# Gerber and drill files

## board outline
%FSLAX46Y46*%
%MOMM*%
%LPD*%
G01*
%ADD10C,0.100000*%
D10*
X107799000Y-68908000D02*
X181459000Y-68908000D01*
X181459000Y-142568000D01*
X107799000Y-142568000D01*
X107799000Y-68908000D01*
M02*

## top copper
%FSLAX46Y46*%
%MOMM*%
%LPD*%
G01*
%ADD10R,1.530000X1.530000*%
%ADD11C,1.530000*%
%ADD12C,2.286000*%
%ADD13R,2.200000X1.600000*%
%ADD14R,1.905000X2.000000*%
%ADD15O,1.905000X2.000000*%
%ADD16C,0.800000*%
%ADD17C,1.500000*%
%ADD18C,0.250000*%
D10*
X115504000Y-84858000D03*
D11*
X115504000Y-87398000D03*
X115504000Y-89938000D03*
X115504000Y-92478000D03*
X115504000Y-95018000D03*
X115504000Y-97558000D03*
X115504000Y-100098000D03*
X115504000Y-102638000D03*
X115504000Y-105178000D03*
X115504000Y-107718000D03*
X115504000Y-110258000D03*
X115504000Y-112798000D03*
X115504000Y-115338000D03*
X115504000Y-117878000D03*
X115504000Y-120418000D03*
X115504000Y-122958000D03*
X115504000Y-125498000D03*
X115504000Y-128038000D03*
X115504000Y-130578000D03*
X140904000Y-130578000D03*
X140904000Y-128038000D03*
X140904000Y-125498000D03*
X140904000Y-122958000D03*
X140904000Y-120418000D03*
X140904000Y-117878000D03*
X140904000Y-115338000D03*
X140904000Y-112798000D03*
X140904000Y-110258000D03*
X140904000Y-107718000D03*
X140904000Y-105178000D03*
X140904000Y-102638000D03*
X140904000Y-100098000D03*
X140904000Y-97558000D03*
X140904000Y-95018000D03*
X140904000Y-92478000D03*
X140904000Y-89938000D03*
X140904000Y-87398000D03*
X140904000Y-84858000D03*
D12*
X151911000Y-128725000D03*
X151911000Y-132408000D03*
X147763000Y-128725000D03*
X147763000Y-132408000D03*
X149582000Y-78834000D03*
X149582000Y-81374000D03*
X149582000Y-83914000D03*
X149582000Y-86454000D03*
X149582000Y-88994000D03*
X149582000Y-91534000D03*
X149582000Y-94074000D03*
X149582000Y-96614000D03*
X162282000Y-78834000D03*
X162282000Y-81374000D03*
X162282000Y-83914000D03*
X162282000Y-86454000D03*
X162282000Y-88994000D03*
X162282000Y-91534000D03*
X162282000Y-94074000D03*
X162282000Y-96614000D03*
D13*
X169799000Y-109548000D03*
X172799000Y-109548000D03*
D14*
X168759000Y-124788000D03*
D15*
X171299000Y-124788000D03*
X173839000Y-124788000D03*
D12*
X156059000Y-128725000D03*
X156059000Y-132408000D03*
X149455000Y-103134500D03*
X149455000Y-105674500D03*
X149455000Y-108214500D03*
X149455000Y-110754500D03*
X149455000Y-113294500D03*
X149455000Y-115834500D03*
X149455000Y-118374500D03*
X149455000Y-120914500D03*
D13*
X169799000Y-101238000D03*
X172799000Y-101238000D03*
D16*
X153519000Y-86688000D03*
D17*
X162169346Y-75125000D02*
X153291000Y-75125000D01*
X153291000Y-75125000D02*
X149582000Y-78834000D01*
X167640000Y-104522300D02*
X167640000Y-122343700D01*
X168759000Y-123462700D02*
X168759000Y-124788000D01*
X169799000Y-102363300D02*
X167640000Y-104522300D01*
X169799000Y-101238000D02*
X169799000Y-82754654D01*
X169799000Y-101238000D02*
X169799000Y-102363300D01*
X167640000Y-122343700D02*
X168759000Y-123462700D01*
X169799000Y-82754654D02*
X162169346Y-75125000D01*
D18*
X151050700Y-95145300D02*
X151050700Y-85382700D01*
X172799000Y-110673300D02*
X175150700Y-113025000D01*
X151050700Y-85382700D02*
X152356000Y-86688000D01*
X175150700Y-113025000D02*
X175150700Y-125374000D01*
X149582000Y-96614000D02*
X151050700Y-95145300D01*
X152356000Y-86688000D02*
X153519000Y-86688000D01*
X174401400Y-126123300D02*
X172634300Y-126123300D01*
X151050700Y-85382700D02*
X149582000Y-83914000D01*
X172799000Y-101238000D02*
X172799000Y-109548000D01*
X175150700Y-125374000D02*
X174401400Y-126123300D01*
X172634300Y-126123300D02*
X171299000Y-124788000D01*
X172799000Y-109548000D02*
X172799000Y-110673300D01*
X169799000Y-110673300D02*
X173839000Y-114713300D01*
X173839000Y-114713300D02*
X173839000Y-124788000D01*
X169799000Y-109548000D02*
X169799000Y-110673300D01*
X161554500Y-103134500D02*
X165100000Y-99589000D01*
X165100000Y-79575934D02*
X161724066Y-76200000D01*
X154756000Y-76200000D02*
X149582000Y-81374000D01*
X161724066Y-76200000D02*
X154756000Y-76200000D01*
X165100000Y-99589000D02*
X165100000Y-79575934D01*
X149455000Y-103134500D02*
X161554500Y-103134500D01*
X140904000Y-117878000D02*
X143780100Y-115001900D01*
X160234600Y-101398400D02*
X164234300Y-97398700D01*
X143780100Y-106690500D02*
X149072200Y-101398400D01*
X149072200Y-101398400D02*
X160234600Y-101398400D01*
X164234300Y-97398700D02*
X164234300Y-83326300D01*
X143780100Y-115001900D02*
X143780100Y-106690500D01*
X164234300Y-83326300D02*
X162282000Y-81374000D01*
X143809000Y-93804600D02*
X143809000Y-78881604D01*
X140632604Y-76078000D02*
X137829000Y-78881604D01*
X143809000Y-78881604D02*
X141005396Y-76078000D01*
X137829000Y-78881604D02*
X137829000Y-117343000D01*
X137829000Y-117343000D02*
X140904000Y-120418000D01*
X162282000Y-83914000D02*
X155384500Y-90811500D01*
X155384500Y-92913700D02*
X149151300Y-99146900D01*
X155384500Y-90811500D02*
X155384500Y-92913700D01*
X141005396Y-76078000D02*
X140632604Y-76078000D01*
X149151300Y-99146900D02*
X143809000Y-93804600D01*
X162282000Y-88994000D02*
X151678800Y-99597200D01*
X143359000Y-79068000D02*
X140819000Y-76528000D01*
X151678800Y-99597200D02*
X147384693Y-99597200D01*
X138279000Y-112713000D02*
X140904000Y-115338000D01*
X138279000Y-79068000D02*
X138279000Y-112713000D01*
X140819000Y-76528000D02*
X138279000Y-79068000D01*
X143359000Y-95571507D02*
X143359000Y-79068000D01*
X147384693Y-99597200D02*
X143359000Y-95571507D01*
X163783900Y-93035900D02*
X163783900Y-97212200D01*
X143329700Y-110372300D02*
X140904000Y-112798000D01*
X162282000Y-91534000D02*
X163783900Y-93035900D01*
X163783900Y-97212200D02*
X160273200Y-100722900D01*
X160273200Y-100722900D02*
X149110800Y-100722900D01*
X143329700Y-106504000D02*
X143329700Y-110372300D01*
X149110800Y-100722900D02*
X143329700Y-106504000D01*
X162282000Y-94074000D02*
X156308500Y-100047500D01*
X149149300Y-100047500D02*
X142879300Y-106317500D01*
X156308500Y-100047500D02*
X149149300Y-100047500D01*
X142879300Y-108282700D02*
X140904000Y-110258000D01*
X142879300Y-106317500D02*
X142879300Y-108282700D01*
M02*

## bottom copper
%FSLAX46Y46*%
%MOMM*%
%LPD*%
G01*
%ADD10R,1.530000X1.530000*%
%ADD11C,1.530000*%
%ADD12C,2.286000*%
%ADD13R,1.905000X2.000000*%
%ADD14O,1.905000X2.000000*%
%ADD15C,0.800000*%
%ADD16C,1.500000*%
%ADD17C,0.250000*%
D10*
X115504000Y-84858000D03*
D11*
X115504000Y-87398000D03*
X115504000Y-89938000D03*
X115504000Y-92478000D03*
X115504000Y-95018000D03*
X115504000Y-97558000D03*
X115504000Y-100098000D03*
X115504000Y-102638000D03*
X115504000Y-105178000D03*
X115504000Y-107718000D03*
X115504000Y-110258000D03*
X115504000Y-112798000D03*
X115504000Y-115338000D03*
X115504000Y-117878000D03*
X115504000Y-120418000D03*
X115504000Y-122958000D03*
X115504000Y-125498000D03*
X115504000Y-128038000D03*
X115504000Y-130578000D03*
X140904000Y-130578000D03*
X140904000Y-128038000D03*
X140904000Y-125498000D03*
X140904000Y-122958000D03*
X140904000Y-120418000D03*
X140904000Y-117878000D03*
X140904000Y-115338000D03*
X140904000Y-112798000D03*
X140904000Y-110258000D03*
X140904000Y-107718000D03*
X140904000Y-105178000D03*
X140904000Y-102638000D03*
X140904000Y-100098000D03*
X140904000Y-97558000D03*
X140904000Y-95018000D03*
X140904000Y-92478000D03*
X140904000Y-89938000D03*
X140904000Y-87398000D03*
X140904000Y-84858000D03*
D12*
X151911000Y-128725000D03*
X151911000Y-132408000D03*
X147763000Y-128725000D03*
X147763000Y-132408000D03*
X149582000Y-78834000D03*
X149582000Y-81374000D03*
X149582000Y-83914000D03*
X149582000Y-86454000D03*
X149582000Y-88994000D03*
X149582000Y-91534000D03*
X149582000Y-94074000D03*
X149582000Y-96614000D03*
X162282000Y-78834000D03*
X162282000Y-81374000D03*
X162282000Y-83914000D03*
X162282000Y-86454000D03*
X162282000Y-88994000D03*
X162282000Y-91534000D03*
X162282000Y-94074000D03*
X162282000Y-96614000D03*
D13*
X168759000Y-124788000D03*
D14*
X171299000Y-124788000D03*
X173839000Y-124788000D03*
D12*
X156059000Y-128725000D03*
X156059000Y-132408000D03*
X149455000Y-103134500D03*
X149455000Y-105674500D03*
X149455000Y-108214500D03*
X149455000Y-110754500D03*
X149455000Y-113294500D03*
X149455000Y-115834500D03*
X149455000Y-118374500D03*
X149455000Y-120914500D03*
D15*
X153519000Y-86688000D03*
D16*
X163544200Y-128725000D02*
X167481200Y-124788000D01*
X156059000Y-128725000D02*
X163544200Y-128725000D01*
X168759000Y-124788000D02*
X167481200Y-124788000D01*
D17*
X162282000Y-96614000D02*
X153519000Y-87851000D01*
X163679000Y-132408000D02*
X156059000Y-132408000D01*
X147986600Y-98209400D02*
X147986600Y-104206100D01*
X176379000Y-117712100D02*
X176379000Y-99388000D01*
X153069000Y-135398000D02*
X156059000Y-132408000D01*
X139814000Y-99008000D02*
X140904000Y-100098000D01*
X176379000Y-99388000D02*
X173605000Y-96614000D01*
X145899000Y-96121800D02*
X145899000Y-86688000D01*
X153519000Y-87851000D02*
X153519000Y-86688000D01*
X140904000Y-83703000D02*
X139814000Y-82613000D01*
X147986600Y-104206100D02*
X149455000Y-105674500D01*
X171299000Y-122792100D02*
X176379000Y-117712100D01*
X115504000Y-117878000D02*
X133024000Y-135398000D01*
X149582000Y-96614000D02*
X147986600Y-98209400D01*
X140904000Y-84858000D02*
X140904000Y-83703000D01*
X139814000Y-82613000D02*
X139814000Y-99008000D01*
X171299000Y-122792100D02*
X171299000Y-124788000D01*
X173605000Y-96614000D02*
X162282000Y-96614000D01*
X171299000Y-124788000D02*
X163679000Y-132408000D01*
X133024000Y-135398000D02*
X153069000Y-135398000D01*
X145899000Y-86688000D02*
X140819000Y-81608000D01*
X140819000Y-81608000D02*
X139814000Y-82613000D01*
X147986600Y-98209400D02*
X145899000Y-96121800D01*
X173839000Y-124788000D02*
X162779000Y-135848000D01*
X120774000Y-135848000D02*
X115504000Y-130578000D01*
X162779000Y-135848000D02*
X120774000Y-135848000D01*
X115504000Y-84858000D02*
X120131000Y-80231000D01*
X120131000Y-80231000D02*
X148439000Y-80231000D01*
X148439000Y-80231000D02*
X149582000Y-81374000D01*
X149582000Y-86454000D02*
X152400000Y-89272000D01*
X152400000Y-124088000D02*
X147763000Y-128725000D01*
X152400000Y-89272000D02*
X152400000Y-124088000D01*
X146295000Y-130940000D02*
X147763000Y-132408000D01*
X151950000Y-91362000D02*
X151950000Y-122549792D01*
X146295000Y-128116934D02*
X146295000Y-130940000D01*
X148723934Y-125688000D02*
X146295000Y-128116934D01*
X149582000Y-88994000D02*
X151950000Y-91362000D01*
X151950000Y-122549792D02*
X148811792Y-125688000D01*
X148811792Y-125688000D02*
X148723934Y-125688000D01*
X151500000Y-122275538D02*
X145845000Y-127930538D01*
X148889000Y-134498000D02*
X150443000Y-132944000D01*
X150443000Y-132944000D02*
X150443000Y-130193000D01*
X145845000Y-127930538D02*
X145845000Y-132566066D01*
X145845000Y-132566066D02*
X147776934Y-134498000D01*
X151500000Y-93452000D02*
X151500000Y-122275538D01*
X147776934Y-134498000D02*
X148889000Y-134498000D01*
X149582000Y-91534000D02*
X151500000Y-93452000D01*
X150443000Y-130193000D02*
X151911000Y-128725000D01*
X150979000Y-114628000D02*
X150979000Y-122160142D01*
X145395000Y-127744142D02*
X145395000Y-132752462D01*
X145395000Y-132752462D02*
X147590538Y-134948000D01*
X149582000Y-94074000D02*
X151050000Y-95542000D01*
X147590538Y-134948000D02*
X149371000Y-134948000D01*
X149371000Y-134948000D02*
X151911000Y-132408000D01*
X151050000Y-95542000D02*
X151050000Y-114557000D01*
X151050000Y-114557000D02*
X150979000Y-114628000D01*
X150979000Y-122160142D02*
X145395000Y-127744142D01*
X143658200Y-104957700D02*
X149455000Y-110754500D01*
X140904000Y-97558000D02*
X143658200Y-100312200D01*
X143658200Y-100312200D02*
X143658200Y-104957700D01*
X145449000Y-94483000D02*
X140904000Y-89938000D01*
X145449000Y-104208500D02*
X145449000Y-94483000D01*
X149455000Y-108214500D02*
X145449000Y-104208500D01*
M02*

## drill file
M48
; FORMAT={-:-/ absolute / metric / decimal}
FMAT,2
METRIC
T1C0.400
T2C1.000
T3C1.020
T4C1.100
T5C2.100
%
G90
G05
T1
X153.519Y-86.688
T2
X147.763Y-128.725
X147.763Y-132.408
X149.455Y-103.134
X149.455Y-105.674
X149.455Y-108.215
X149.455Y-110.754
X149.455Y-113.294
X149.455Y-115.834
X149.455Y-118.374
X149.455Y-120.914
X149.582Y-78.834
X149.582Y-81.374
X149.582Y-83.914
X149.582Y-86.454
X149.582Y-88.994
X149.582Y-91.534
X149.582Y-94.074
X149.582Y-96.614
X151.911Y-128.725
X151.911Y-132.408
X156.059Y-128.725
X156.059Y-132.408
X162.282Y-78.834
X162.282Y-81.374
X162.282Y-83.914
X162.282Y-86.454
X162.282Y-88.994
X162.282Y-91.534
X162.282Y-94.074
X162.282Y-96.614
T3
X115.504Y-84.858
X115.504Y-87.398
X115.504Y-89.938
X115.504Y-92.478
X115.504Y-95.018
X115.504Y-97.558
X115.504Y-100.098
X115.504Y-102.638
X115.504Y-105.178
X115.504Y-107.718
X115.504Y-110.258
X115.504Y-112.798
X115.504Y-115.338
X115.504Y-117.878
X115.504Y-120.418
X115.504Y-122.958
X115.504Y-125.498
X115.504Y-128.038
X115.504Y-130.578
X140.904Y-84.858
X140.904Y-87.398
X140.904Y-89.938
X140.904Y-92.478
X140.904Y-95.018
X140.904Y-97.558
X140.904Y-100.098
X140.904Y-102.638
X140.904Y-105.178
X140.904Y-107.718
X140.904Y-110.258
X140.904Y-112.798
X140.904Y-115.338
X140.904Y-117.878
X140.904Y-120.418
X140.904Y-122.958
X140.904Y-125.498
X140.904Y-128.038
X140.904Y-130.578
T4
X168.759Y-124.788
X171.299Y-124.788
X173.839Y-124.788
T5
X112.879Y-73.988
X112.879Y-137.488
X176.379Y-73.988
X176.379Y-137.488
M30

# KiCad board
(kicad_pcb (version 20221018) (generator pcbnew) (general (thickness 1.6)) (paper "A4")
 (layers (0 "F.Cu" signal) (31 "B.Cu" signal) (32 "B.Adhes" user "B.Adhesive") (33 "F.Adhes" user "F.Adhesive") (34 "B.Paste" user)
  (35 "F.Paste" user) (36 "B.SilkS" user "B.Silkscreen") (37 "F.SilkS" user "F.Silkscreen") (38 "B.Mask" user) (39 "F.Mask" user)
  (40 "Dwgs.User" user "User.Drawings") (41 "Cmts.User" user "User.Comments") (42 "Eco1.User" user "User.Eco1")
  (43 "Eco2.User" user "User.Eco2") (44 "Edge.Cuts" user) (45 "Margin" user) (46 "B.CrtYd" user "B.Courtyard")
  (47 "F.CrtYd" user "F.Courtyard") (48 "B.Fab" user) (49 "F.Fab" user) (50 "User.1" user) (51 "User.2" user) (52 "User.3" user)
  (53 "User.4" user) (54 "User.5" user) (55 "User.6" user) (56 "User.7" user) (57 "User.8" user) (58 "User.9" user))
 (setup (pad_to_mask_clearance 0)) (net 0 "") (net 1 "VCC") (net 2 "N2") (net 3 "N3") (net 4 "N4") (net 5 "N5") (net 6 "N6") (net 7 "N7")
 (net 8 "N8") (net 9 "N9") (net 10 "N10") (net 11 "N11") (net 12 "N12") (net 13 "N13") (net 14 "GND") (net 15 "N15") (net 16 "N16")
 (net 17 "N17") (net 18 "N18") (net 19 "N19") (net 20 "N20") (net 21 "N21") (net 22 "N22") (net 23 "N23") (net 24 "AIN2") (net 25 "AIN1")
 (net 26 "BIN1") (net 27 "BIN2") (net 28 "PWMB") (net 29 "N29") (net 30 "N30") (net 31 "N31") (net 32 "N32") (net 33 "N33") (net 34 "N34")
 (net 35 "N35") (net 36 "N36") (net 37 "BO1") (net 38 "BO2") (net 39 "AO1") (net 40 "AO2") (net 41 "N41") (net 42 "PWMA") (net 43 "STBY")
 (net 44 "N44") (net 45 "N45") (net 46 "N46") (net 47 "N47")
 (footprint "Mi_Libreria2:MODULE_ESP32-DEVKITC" (layer "F.Cu") (at 128.204 107.708)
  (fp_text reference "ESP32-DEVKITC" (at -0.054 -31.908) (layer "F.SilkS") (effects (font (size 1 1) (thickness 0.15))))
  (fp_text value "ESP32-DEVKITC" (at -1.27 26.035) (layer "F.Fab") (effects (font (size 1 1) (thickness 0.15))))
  (pad "1" thru_hole rect (at -12.7 -22.85) (size 1.53 1.53) (drill 1.02) (layers "*.Cu" "*.Mask") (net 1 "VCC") (solder_mask_margin 0.102))
  (pad "2" thru_hole circle (at -12.7 -20.31) (size 1.53 1.53) (drill 1.02) (layers "*.Cu" "*.Mask") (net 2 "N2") (solder_mask_margin 0.102))
  (pad "3" thru_hole circle (at -12.7 -17.77) (size 1.53 1.53) (drill 1.02) (layers "*.Cu" "*.Mask") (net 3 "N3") (solder_mask_margin 0.102))
  (pad "4" thru_hole circle (at -12.7 -15.23) (size 1.53 1.53) (drill 1.02) (layers "*.Cu" "*.Mask") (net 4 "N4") (solder_mask_margin 0.102))
  (pad "5" thru_hole circle (at -12.7 -12.69) (size 1.53 1.53) (drill 1.02) (layers "*.Cu" "*.Mask") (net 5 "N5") (solder_mask_margin 0.102))
  (pad "6" thru_hole circle (at -12.7 -10.15) (size 1.53 1.53) (drill 1.02) (layers "*.Cu" "*.Mask") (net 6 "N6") (solder_mask_margin 0.102))
  (pad "7" thru_hole circle (at -12.7 -7.61) (size 1.53 1.53) (drill 1.02) (layers "*.Cu" "*.Mask") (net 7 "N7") (solder_mask_margin 0.102))
  (pad "8" thru_hole circle (at -12.7 -5.07) (size 1.53 1.53) (drill 1.02) (layers "*.Cu" "*.Mask") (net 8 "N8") (solder_mask_margin 0.102))
  (pad "9" thru_hole circle (at -12.7 -2.53) (size 1.53 1.53) (drill 1.02) (layers "*.Cu" "*.Mask") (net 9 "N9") (solder_mask_margin 0.102))
  (pad "10" thru_hole circle (at -12.7 0.01) (size 1.53 1.53) (drill 1.02) (layers "*.Cu" "*.Mask") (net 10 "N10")
   (solder_mask_margin 0.102))
  (pad "11" thru_hole circle (at -12.7 2.55) (size 1.53 1.53) (drill 1.02) (layers "*.Cu" "*.Mask") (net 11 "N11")
   (solder_mask_margin 0.102))
  (pad "12" thru_hole circle (at -12.7 5.09) (size 1.53 1.53) (drill 1.02) (layers "*.Cu" "*.Mask") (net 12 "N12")
   (solder_mask_margin 0.102))
  (pad "13" thru_hole circle (at -12.7 7.63) (size 1.53 1.53) (drill 1.02) (layers "*.Cu" "*.Mask") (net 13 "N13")
   (solder_mask_margin 0.102))
  (pad "14" thru_hole circle (at -12.7 10.17) (size 1.53 1.53) (drill 1.02) (layers "*.Cu" "*.Mask") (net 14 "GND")
   (solder_mask_margin 0.102))
  (pad "15" thru_hole circle (at -12.7 12.71) (size 1.53 1.53) (drill 1.02) (layers "*.Cu" "*.Mask") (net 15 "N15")
   (solder_mask_margin 0.102))
  (pad "16" thru_hole circle (at -12.7 15.25) (size 1.53 1.53) (drill 1.02) (layers "*.Cu" "*.Mask") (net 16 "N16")
   (solder_mask_margin 0.102))
  (pad "17" thru_hole circle (at -12.7 17.79) (size 1.53 1.53) (drill 1.02) (layers "*.Cu" "*.Mask") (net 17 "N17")
   (solder_mask_margin 0.102))
  (pad "18" thru_hole circle (at -12.7 20.33) (size 1.53 1.53) (drill 1.02) (layers "*.Cu" "*.Mask") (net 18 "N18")
   (solder_mask_margin 0.102))
  (pad "19" thru_hole circle (at -12.7 22.87) (size 1.53 1.53) (drill 1.02) (layers "*.Cu" "*.Mask") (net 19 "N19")
   (solder_mask_margin 0.102))
  (pad "20" thru_hole circle (at 12.7 22.87) (size 1.53 1.53) (drill 1.02) (layers "*.Cu" "*.Mask") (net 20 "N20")
   (solder_mask_margin 0.102))
  (pad "21" thru_hole circle (at 12.7 20.33) (size 1.53 1.53) (drill 1.02) (layers "*.Cu" "*.Mask") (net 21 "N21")
   (solder_mask_margin 0.102))
  (pad "22" thru_hole circle (at 12.7 17.79) (size 1.53 1.53) (drill 1.02) (layers "*.Cu" "*.Mask") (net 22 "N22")
   (solder_mask_margin 0.102))
  (pad "23" thru_hole circle (at 12.7 15.25) (size 1.53 1.53) (drill 1.02) (layers "*.Cu" "*.Mask") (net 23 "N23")
   (solder_mask_margin 0.102))
  (pad "24" thru_hole circle (at 12.7 12.71) (size 1.53 1.53) (drill 1.02) (layers "*.Cu" "*.Mask") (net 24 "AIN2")
   (solder_mask_margin 0.102))
  (pad "25" thru_hole circle (at 12.7 10.17) (size 1.53 1.53) (drill 1.02) (layers "*.Cu" "*.Mask") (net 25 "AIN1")
   (solder_mask_margin 0.102))
  (pad "26" thru_hole circle (at 12.7 7.63) (size 1.53 1.53) (drill 1.02) (layers "*.Cu" "*.Mask") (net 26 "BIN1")
   (solder_mask_margin 0.102))
  (pad "27" thru_hole circle (at 12.7 5.09) (size 1.53 1.53) (drill 1.02) (layers "*.Cu" "*.Mask") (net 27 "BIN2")
   (solder_mask_margin 0.102))
  (pad "28" thru_hole circle (at 12.7 2.55) (size 1.53 1.53) (drill 1.02) (layers "*.Cu" "*.Mask") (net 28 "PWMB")
   (solder_mask_margin 0.102))
  (pad "29" thru_hole circle (at 12.7 0.01) (size 1.53 1.53) (drill 1.02) (layers "*.Cu" "*.Mask") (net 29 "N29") (solder_mask_margin 0.102))
  (pad "30" thru_hole circle (at 12.7 -2.53) (size 1.53 1.53) (drill 1.02) (layers "*.Cu" "*.Mask") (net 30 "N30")
   (solder_mask_margin 0.102))
  (pad "31" thru_hole circle (at 12.7 -5.07) (size 1.53 1.53) (drill 1.02) (layers "*.Cu" "*.Mask") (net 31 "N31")
   (solder_mask_margin 0.102))
  (pad "32" thru_hole circle (at 12.7 -7.61) (size 1.53 1.53) (drill 1.02) (layers "*.Cu" "*.Mask") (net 14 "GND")
   (solder_mask_margin 0.102))
  (pad "33" thru_hole circle (at 12.7 -10.15) (size 1.53 1.53) (drill 1.02) (layers "*.Cu" "*.Mask") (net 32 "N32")
   (solder_mask_margin 0.102))
  (pad "34" thru_hole circle (at 12.7 -12.69) (size 1.53 1.53) (drill 1.02) (layers "*.Cu" "*.Mask") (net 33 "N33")
   (solder_mask_margin 0.102))
  (pad "35" thru_hole circle (at 12.7 -15.23) (size 1.53 1.53) (drill 1.02) (layers "*.Cu" "*.Mask") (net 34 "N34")
   (solder_mask_margin 0.102))
  (pad "36" thru_hole circle (at 12.7 -17.77) (size 1.53 1.53) (drill 1.02) (layers "*.Cu" "*.Mask") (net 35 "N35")
   (solder_mask_margin 0.102))
  (pad "37" thru_hole circle (at 12.7 -20.31) (size 1.53 1.53) (drill 1.02) (layers "*.Cu" "*.Mask") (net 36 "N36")
   (solder_mask_margin 0.102))
  (pad "38" thru_hole circle (at 12.7 -22.85) (size 1.53 1.53) (drill 1.02) (layers "*.Cu" "*.Mask") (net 14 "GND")
   (solder_mask_margin 0.102)))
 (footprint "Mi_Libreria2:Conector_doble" (layer "F.Cu") (at 151.911 128.725)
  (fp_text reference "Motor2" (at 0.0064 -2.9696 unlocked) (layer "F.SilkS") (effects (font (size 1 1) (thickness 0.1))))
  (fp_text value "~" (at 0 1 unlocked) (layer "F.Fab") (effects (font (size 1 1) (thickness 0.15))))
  (pad "1" thru_hole circle (at 0 0) (size 2.286 2.286) (drill 1) (layers "*.Cu" "*.Mask") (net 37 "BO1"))
  (pad "2" thru_hole circle (at 0 3.683) (size 2.286 2.286) (drill 1) (layers "*.Cu" "*.Mask") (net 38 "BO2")))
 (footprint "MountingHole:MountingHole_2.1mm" (layer "F.Cu") (at 112.879 137.488)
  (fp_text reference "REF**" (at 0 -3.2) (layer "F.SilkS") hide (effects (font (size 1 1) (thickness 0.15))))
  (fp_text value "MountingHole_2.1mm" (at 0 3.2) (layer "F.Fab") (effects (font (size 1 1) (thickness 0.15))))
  (pad "" np_thru_hole circle (at 0 0) (size 2.1 2.1) (drill 2.1) (layers "F&B.Cu" "*.Mask")))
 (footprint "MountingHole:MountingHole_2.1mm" (layer "F.Cu") (at 112.879 73.988)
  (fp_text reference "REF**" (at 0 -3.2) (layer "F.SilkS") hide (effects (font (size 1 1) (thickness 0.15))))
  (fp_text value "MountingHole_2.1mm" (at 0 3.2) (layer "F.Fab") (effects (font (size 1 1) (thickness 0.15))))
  (pad "" np_thru_hole circle (at 0 0) (size 2.1 2.1) (drill 2.1) (layers "F&B.Cu" "*.Mask")))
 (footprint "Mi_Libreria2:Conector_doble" (layer "F.Cu") (at 147.763 128.725)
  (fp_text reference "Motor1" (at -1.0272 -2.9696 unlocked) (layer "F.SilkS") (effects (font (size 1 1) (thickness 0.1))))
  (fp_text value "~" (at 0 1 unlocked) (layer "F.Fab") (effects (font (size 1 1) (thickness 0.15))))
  (pad "1" thru_hole circle (at 0 0) (size 2.286 2.286) (drill 1) (layers "*.Cu" "*.Mask") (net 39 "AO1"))
  (pad "2" thru_hole circle (at 0 3.683) (size 2.286 2.286) (drill 1) (layers "*.Cu" "*.Mask") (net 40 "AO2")))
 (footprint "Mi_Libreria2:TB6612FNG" (layer "F.Cu") (at 149.582 78.834)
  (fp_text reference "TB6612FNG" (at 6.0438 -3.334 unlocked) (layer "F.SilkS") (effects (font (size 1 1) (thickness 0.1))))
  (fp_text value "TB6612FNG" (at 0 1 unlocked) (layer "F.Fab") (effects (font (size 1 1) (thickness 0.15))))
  (pad "1" thru_hole circle (at 0 0) (size 2.286 2.286) (drill 1) (layers "*.Cu" "*.Mask") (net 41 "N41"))
  (pad "2" thru_hole circle (at 0 2.54) (size 2.286 2.286) (drill 1) (layers "*.Cu" "*.Mask") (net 1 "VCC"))
  (pad "3" thru_hole circle (at 0 5.08) (size 2.286 2.286) (drill 1) (layers "*.Cu" "*.Mask") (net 14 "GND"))
  (pad "4" thru_hole circle (at 0 7.62) (size 2.286 2.286) (drill 1) (layers "*.Cu" "*.Mask") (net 39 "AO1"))
  (pad "5" thru_hole circle (at 0 10.16) (size 2.286 2.286) (drill 1) (layers "*.Cu" "*.Mask") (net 40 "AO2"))
  (pad "6" thru_hole circle (at 0 12.7) (size 2.286 2.286) (drill 1) (layers "*.Cu" "*.Mask") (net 37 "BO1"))
  (pad "7" thru_hole circle (at 0 15.24) (size 2.286 2.286) (drill 1) (layers "*.Cu" "*.Mask") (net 38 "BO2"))
  (pad "8" thru_hole circle (at 0 17.78) (size 2.286 2.286) (drill 1) (layers "*.Cu" "*.Mask") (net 14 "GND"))
  (pad "9" thru_hole circle (at 12.7 0) (size 2.286 2.286) (drill 1) (layers "*.Cu" "*.Mask") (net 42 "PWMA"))
  (pad "10" thru_hole circle (at 12.7 2.54) (size 2.286 2.286) (drill 1) (layers "*.Cu" "*.Mask") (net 25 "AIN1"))
  (pad "11" thru_hole circle (at 12.7 5.08) (size 2.286 2.286) (drill 1) (layers "*.Cu" "*.Mask") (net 24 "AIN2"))
  (pad "12" thru_hole circle (at 12.7 7.62) (size 2.286 2.286) (drill 1) (layers "*.Cu" "*.Mask") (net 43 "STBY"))
  (pad "13" thru_hole circle (at 12.7 10.16) (size 2.286 2.286) (drill 1) (layers "*.Cu" "*.Mask") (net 26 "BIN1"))
  (pad "14" thru_hole circle (at 12.7 12.7) (size 2.286 2.286) (drill 1) (layers "*.Cu" "*.Mask") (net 27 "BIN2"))
  (pad "15" thru_hole circle (at 12.7 15.24) (size 2.286 2.286) (drill 1) (layers "*.Cu" "*.Mask") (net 28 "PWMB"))
  (pad "16" thru_hole circle (at 12.7 17.78) (size 2.286 2.286) (drill 1) (layers "*.Cu" "*.Mask") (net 14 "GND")))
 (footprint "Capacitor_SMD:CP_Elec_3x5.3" (layer "F.Cu") (at 171.299 109.548)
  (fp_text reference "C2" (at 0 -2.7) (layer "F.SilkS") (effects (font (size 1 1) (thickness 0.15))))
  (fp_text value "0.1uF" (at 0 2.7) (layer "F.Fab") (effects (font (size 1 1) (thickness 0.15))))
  (pad "1" smd rect (at -1.5 0) (size 2.2 1.6) (layers "F.Cu" "F.Paste" "F.Mask") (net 19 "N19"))
  (pad "2" smd rect (at 1.5 0) (size 2.2 1.6) (layers "F.Cu" "F.Paste" "F.Mask") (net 14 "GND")))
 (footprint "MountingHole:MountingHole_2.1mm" (layer "F.Cu") (at 176.379 137.488)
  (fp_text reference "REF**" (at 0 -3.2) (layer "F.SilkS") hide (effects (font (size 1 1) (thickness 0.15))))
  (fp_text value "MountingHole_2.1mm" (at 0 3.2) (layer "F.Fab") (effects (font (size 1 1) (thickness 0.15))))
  (pad "" np_thru_hole circle (at 0 0) (size 2.1 2.1) (drill 2.1) (layers "F&B.Cu" "*.Mask")))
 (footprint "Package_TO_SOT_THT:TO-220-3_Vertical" (layer "F.Cu") (at 168.759 124.788)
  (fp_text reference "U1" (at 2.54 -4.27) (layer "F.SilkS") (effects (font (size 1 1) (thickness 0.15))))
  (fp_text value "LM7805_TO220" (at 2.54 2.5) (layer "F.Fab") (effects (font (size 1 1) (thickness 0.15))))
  (pad "1" thru_hole rect (at 0 0) (size 1.905 2) (drill 1.1) (layers "*.Cu" "*.Mask") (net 41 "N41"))
  (pad "2" thru_hole oval (at 2.54 0) (size 1.905 2) (drill 1.1) (layers "*.Cu" "*.Mask") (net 14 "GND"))
  (pad "3" thru_hole oval (at 5.08 0) (size 1.905 2) (drill 1.1) (layers "*.Cu" "*.Mask") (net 19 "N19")))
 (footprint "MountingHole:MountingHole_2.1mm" (layer "F.Cu") (at 176.379 73.988)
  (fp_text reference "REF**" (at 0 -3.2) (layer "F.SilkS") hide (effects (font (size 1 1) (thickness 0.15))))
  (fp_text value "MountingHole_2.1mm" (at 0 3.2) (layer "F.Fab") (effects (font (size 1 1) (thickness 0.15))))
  (pad "" np_thru_hole circle (at 0 0) (size 2.1 2.1) (drill 2.1) (layers "F&B.Cu" "*.Mask")))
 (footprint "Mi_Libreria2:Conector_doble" (layer "F.Cu") (at 156.059 128.725)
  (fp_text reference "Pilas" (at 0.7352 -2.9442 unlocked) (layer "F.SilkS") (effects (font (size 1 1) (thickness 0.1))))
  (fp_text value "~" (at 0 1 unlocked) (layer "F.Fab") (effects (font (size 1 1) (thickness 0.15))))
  (pad "1" thru_hole circle (at 0 0) (size 2.286 2.286) (drill 1) (layers "*.Cu" "*.Mask") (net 41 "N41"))
  (pad "2" thru_hole circle (at 0 3.683) (size 2.286 2.286) (drill 1) (layers "*.Cu" "*.Mask") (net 14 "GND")))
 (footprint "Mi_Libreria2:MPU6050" (layer "F.Cu") (at 149.455 103.1345)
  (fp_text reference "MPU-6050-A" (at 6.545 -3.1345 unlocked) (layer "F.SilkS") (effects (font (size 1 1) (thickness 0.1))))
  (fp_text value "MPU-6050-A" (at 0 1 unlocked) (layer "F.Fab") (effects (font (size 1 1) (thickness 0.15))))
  (pad "1" thru_hole circle (at 0 0) (size 2.286 2.286) (drill 1) (layers "*.Cu" "*.Mask") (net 1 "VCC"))
  (pad "2" thru_hole circle (at 0 2.54) (size 2.286 2.286) (drill 1) (layers "*.Cu" "*.Mask") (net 14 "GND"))
  (pad "3" thru_hole circle (at 0 5.08) (size 2.286 2.286) (drill 1) (layers "*.Cu" "*.Mask") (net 35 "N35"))
  (pad "4" thru_hole circle (at 0 7.62) (size 2.286 2.286) (drill 1) (layers "*.Cu" "*.Mask") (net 32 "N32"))
  (pad "5" thru_hole circle (at 0 10.16) (size 2.286 2.286) (drill 1) (layers "*.Cu" "*.Mask") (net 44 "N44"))
  (pad "6" thru_hole circle (at 0 12.7) (size 2.286 2.286) (drill 1) (layers "*.Cu" "*.Mask") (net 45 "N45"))
  (pad "7" thru_hole circle (at 0 15.24) (size 2.286 2.286) (drill 1) (layers "*.Cu" "*.Mask") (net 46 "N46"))
  (pad "8" thru_hole circle (at 0 17.78) (size 2.286 2.286) (drill 1) (layers "*.Cu" "*.Mask") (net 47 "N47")))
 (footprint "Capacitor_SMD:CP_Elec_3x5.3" (layer "F.Cu") (at 171.299 101.238)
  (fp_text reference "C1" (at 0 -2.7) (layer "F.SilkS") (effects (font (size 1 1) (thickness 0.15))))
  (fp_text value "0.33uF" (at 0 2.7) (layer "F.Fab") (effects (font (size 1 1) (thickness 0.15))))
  (pad "1" smd rect (at -1.5 0) (size 2.2 1.6) (layers "F.Cu" "F.Paste" "F.Mask") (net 41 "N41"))
  (pad "2" smd rect (at 1.5 0) (size 2.2 1.6) (layers "F.Cu" "F.Paste" "F.Mask") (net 14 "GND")))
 (gr_rect (start 107.799 68.908) (end 181.459 142.568) (stroke (width 0.1) (type default)) (fill none) (layer "Edge.Cuts"))
 (segment (start 162.169346 75.125) (end 153.291 75.125) (width 1.5) (layer "F.Cu") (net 41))
 (segment (start 153.291 75.125) (end 149.582 78.834) (width 1.5) (layer "F.Cu") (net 41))
 (segment (start 167.64 104.5223) (end 167.64 122.3437) (width 1.5) (layer "F.Cu") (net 41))
 (segment (start 168.759 123.4627) (end 168.759 124.788) (width 1.5) (layer "F.Cu") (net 41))
 (segment (start 169.799 102.3633) (end 167.64 104.5223) (width 1.5) (layer "F.Cu") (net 41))
 (segment (start 169.799 101.238) (end 169.799 82.754654) (width 1.5) (layer "F.Cu") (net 41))
 (segment (start 169.799 101.238) (end 169.799 102.3633) (width 1.5) (layer "F.Cu") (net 41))
 (segment (start 167.64 122.3437) (end 168.759 123.4627) (width 1.5) (layer "F.Cu") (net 41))
 (segment (start 169.799 82.754654) (end 162.169346 75.125) (width 1.5) (layer "F.Cu") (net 41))
 (segment (start 163.5442 128.725) (end 167.4812 124.788) (width 1.5) (layer "B.Cu") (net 41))
 (segment (start 156.059 128.725) (end 163.5442 128.725) (width 1.5) (layer "B.Cu") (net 41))
 (segment (start 168.759 124.788) (end 167.4812 124.788) (width 1.5) (layer "B.Cu") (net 41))
 (segment (start 151.0507 95.1453) (end 151.0507 85.3827) (width 0.25) (layer "F.Cu") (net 14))
 (segment (start 172.799 110.6733) (end 175.1507 113.025) (width 0.25) (layer "F.Cu") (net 14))
 (segment (start 151.0507 85.3827) (end 152.356 86.688) (width 0.25) (layer "F.Cu") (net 14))
 (segment (start 175.1507 113.025) (end 175.1507 125.374) (width 0.25) (layer "F.Cu") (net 14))
 (segment (start 149.582 96.614) (end 151.0507 95.1453) (width 0.25) (layer "F.Cu") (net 14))
 (segment (start 152.356 86.688) (end 153.519 86.688) (width 0.25) (layer "F.Cu") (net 14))
 (segment (start 174.4014 126.1233) (end 172.6343 126.1233) (width 0.25) (layer "F.Cu") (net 14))
 (segment (start 151.0507 85.3827) (end 149.582 83.914) (width 0.25) (layer "F.Cu") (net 14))
 (segment (start 172.799 101.238) (end 172.799 109.548) (width 0.25) (layer "F.Cu") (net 14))
 (segment (start 175.1507 125.374) (end 174.4014 126.1233) (width 0.25) (layer "F.Cu") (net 14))
 (segment (start 172.6343 126.1233) (end 171.299 124.788) (width 0.25) (layer "F.Cu") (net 14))
 (segment (start 172.799 109.548) (end 172.799 110.6733) (width 0.25) (layer "F.Cu") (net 14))
 (via (at 153.519 86.688) (size 0.8) (drill 0.4) (layers "F.Cu" "B.Cu") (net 14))
 (segment (start 162.282 96.614) (end 153.519 87.851) (width 0.25) (layer "B.Cu") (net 14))
 (segment (start 163.679 132.408) (end 156.059 132.408) (width 0.25) (layer "B.Cu") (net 14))
 (segment (start 147.9866 98.2094) (end 147.9866 104.2061) (width 0.25) (layer "B.Cu") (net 14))
 (segment (start 176.379 117.7121) (end 176.379 99.388) (width 0.25) (layer "B.Cu") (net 14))
 (segment (start 153.069 135.398) (end 156.059 132.408) (width 0.25) (layer "B.Cu") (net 14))
 (segment (start 139.814 99.008) (end 140.904 100.098) (width 0.25) (layer "B.Cu") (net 14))
 (segment (start 176.379 99.388) (end 173.605 96.614) (width 0.25) (layer "B.Cu") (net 14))
 (segment (start 145.899 96.1218) (end 145.899 86.688) (width 0.25) (layer "B.Cu") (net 14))
 (segment (start 153.519 87.851) (end 153.519 86.688) (width 0.25) (layer "B.Cu") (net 14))
 (segment (start 140.904 83.703) (end 139.814 82.613) (width 0.25) (layer "B.Cu") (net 14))
 (segment (start 147.9866 104.2061) (end 149.455 105.6745) (width 0.25) (layer "B.Cu") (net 14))
 (segment (start 171.299 122.7921) (end 176.379 117.7121) (width 0.25) (layer "B.Cu") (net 14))
 (segment (start 115.504 117.878) (end 133.024 135.398) (width 0.25) (layer "B.Cu") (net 14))
 (segment (start 149.582 96.614) (end 147.9866 98.2094) (width 0.25) (layer "B.Cu") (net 14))
 (segment (start 140.904 84.858) (end 140.904 83.703) (width 0.25) (layer "B.Cu") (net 14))
 (segment (start 139.814 82.613) (end 139.814 99.008) (width 0.25) (layer "B.Cu") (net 14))
 (segment (start 171.299 122.7921) (end 171.299 124.788) (width 0.25) (layer "B.Cu") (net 14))
 (segment (start 173.605 96.614) (end 162.282 96.614) (width 0.25) (layer "B.Cu") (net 14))
 (segment (start 171.299 124.788) (end 163.679 132.408) (width 0.25) (layer "B.Cu") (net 14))
 (segment (start 133.024 135.398) (end 153.069 135.398) (width 0.25) (layer "B.Cu") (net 14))
 (segment (start 145.899 86.688) (end 140.819 81.608) (width 0.25) (layer "B.Cu") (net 14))
 (segment (start 140.819 81.608) (end 139.814 82.613) (width 0.25) (layer "B.Cu") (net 14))
 (segment (start 147.9866 98.2094) (end 145.899 96.1218) (width 0.25) (layer "B.Cu") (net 14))
 (segment (start 169.799 110.6733) (end 173.839 114.7133) (width 0.25) (layer "F.Cu") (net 19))
 (segment (start 173.839 114.7133) (end 173.839 124.788) (width 0.25) (layer "F.Cu") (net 19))
 (segment (start 169.799 109.548) (end 169.799 110.6733) (width 0.25) (layer "F.Cu") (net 19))
 (segment (start 173.839 124.788) (end 162.779 135.848) (width 0.25) (layer "B.Cu") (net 19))
 (segment (start 120.774 135.848) (end 115.504 130.578) (width 0.25) (layer "B.Cu") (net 19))
 (segment (start 162.779 135.848) (end 120.774 135.848) (width 0.25) (layer "B.Cu") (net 19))
 (segment (start 161.5545 103.1345) (end 165.1 99.589) (width 0.25) (layer "F.Cu") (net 1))
 (segment (start 165.1 79.575934) (end 161.724066 76.2) (width 0.25) (layer "F.Cu") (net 1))
 (segment (start 154.756 76.2) (end 149.582 81.374) (width 0.25) (layer "F.Cu") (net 1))
 (segment (start 161.724066 76.2) (end 154.756 76.2) (width 0.25) (layer "F.Cu") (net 1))
 (segment (start 165.1 99.589) (end 165.1 79.575934) (width 0.25) (layer "F.Cu") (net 1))
 (segment (start 149.455 103.1345) (end 161.5545 103.1345) (width 0.25) (layer "F.Cu") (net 1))
 (segment (start 115.504 84.858) (end 120.131 80.231) (width 0.25) (layer "B.Cu") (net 1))
 (segment (start 120.131 80.231) (end 148.439 80.231) (width 0.25) (layer "B.Cu") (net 1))
 (segment (start 148.439 80.231) (end 149.582 81.374) (width 0.25) (layer "B.Cu") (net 1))
 (segment (start 149.582 86.454) (end 152.4 89.272) (width 0.25) (layer "B.Cu") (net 39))
 (segment (start 152.4 124.088) (end 147.763 128.725) (width 0.25) (layer "B.Cu") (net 39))
 (segment (start 152.4 89.272) (end 152.4 124.088) (width 0.25) (layer "B.Cu") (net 39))
 (segment (start 146.295 130.94) (end 147.763 132.408) (width 0.25) (layer "B.Cu") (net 40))
 (segment (start 151.95 91.362) (end 151.95 122.549792) (width 0.25) (layer "B.Cu") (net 40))
 (segment (start 146.295 128.116934) (end 146.295 130.94) (width 0.25) (layer "B.Cu") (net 40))
 (segment (start 148.723934 125.688) (end 146.295 128.116934) (width 0.25) (layer "B.Cu") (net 40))
 (segment (start 149.582 88.994) (end 151.95 91.362) (width 0.25) (layer "B.Cu") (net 40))
 (segment (start 151.95 122.549792) (end 148.811792 125.688) (width 0.25) (layer "B.Cu") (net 40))
 (segment (start 148.811792 125.688) (end 148.723934 125.688) (width 0.25) (layer "B.Cu") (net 40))
 (segment (start 151.5 122.275538) (end 145.845 127.930538) (width 0.25) (layer "B.Cu") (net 37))
 (segment (start 148.889 134.498) (end 150.443 132.944) (width 0.25) (layer "B.Cu") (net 37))
 (segment (start 150.443 132.944) (end 150.443 130.193) (width 0.25) (layer "B.Cu") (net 37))
 (segment (start 145.845 127.930538) (end 145.845 132.566066) (width 0.25) (layer "B.Cu") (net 37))
 (segment (start 145.845 132.566066) (end 147.776934 134.498) (width 0.25) (layer "B.Cu") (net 37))
 (segment (start 151.5 93.452) (end 151.5 122.275538) (width 0.25) (layer "B.Cu") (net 37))
 (segment (start 147.776934 134.498) (end 148.889 134.498) (width 0.25) (layer "B.Cu") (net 37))
 (segment (start 149.582 91.534) (end 151.5 93.452) (width 0.25) (layer "B.Cu") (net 37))
 (segment (start 150.443 130.193) (end 151.911 128.725) (width 0.25) (layer "B.Cu") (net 37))
 (segment (start 150.979 114.628) (end 150.979 122.160142) (width 0.25) (layer "B.Cu") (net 38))
 (segment (start 145.395 127.744142) (end 145.395 132.752462) (width 0.25) (layer "B.Cu") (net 38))
 (segment (start 145.395 132.752462) (end 147.590538 134.948) (width 0.25) (layer "B.Cu") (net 38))
 (segment (start 149.582 94.074) (end 151.05 95.542) (width 0.25) (layer "B.Cu") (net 38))
 (segment (start 147.590538 134.948) (end 149.371 134.948) (width 0.25) (layer "B.Cu") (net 38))
 (segment (start 149.371 134.948) (end 151.911 132.408) (width 0.25) (layer "B.Cu") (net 38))
 (segment (start 151.05 95.542) (end 151.05 114.557) (width 0.25) (layer "B.Cu") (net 38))
 (segment (start 151.05 114.557) (end 150.979 114.628) (width 0.25) (layer "B.Cu") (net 38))
 (segment (start 150.979 122.160142) (end 145.395 127.744142) (width 0.25) (layer "B.Cu") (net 38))
 (segment (start 140.904 117.878) (end 143.7801 115.0019) (width 0.25) (layer "F.Cu") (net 25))
 (segment (start 160.2346 101.3984) (end 164.2343 97.3987) (width 0.25) (layer "F.Cu") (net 25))
 (segment (start 143.7801 106.6905) (end 149.0722 101.3984) (width 0.25) (layer "F.Cu") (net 25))
 (segment (start 149.0722 101.3984) (end 160.2346 101.3984) (width 0.25) (layer "F.Cu") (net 25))
 (segment (start 164.2343 97.3987) (end 164.2343 83.3263) (width 0.25) (layer "F.Cu") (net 25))
 (segment (start 143.7801 115.0019) (end 143.7801 106.6905) (width 0.25) (layer "F.Cu") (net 25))
 (segment (start 164.2343 83.3263) (end 162.282 81.374) (width 0.25) (layer "F.Cu") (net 25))
 (segment (start 143.809 93.8046) (end 143.809 78.881604) (width 0.25) (layer "F.Cu") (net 24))
 (segment (start 140.632604 76.078) (end 137.829 78.881604) (width 0.25) (layer "F.Cu") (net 24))
 (segment (start 143.809 78.881604) (end 141.005396 76.078) (width 0.25) (layer "F.Cu") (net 24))
 (segment (start 137.829 78.881604) (end 137.829 117.343) (width 0.25) (layer "F.Cu") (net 24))
 (segment (start 137.829 117.343) (end 140.904 120.418) (width 0.25) (layer "F.Cu") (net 24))
 (segment (start 162.282 83.914) (end 155.3845 90.8115) (width 0.25) (layer "F.Cu") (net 24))
 (segment (start 155.3845 92.9137) (end 149.1513 99.1469) (width 0.25) (layer "F.Cu") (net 24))
 (segment (start 155.3845 90.8115) (end 155.3845 92.9137) (width 0.25) (layer "F.Cu") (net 24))
 (segment (start 141.005396 76.078) (end 140.632604 76.078) (width 0.25) (layer "F.Cu") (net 24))
 (segment (start 149.1513 99.1469) (end 143.809 93.8046) (width 0.25) (layer "F.Cu") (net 24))
 (segment (start 162.282 88.994) (end 151.6788 99.5972) (width 0.25) (layer "F.Cu") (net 26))
 (segment (start 143.359 79.068) (end 140.819 76.528) (width 0.25) (layer "F.Cu") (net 26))
 (segment (start 151.6788 99.5972) (end 147.384693 99.5972) (width 0.25) (layer "F.Cu") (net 26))
 (segment (start 138.279 112.713) (end 140.904 115.338) (width 0.25) (layer "F.Cu") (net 26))
 (segment (start 138.279 79.068) (end 138.279 112.713) (width 0.25) (layer "F.Cu") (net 26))
 (segment (start 140.819 76.528) (end 138.279 79.068) (width 0.25) (layer "F.Cu") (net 26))
 (segment (start 143.359 95.571507) (end 143.359 79.068) (width 0.25) (layer "F.Cu") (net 26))
 (segment (start 147.384693 99.5972) (end 143.359 95.571507) (width 0.25) (layer "F.Cu") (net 26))
 (segment (start 163.7839 93.0359) (end 163.7839 97.2122) (width 0.25) (layer "F.Cu") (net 27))
 (segment (start 143.3297 110.3723) (end 140.904 112.798) (width 0.25) (layer "F.Cu") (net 27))
 (segment (start 162.282 91.534) (end 163.7839 93.0359) (width 0.25) (layer "F.Cu") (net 27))
 (segment (start 163.7839 97.2122) (end 160.2732 100.7229) (width 0.25) (layer "F.Cu") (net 27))
 (segment (start 160.2732 100.7229) (end 149.1108 100.7229) (width 0.25) (layer "F.Cu") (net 27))
 (segment (start 143.3297 106.504) (end 143.3297 110.3723) (width 0.25) (layer "F.Cu") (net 27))
 (segment (start 149.1108 100.7229) (end 143.3297 106.504) (width 0.25) (layer "F.Cu") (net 27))
 (segment (start 162.282 94.074) (end 156.3085 100.0475) (width 0.25) (layer "F.Cu") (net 28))
 (segment (start 149.1493 100.0475) (end 142.8793 106.3175) (width 0.25) (layer "F.Cu") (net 28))
 (segment (start 156.3085 100.0475) (end 149.1493 100.0475) (width 0.25) (layer "F.Cu") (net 28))
 (segment (start 142.8793 108.2827) (end 140.904 110.258) (width 0.25) (layer "F.Cu") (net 28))
 (segment (start 142.8793 106.3175) (end 142.8793 108.2827) (width 0.25) (layer "F.Cu") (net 28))
 (segment (start 143.6582 104.9577) (end 149.455 110.7545) (width 0.25) (layer "B.Cu") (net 32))
 (segment (start 140.904 97.558) (end 143.6582 100.3122) (width 0.25) (layer "B.Cu") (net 32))
 (segment (start 143.6582 100.3122) (end 143.6582 104.9577) (width 0.25) (layer "B.Cu") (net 32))
 (segment (start 145.449 94.483) (end 140.904 89.938) (width 0.25) (layer "B.Cu") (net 35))
 (segment (start 145.449 104.2085) (end 145.449 94.483) (width 0.25) (layer "B.Cu") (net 35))
 (segment (start 149.455 108.2145) (end 145.449 104.2085) (width 0.25) (layer "B.Cu") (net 35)))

